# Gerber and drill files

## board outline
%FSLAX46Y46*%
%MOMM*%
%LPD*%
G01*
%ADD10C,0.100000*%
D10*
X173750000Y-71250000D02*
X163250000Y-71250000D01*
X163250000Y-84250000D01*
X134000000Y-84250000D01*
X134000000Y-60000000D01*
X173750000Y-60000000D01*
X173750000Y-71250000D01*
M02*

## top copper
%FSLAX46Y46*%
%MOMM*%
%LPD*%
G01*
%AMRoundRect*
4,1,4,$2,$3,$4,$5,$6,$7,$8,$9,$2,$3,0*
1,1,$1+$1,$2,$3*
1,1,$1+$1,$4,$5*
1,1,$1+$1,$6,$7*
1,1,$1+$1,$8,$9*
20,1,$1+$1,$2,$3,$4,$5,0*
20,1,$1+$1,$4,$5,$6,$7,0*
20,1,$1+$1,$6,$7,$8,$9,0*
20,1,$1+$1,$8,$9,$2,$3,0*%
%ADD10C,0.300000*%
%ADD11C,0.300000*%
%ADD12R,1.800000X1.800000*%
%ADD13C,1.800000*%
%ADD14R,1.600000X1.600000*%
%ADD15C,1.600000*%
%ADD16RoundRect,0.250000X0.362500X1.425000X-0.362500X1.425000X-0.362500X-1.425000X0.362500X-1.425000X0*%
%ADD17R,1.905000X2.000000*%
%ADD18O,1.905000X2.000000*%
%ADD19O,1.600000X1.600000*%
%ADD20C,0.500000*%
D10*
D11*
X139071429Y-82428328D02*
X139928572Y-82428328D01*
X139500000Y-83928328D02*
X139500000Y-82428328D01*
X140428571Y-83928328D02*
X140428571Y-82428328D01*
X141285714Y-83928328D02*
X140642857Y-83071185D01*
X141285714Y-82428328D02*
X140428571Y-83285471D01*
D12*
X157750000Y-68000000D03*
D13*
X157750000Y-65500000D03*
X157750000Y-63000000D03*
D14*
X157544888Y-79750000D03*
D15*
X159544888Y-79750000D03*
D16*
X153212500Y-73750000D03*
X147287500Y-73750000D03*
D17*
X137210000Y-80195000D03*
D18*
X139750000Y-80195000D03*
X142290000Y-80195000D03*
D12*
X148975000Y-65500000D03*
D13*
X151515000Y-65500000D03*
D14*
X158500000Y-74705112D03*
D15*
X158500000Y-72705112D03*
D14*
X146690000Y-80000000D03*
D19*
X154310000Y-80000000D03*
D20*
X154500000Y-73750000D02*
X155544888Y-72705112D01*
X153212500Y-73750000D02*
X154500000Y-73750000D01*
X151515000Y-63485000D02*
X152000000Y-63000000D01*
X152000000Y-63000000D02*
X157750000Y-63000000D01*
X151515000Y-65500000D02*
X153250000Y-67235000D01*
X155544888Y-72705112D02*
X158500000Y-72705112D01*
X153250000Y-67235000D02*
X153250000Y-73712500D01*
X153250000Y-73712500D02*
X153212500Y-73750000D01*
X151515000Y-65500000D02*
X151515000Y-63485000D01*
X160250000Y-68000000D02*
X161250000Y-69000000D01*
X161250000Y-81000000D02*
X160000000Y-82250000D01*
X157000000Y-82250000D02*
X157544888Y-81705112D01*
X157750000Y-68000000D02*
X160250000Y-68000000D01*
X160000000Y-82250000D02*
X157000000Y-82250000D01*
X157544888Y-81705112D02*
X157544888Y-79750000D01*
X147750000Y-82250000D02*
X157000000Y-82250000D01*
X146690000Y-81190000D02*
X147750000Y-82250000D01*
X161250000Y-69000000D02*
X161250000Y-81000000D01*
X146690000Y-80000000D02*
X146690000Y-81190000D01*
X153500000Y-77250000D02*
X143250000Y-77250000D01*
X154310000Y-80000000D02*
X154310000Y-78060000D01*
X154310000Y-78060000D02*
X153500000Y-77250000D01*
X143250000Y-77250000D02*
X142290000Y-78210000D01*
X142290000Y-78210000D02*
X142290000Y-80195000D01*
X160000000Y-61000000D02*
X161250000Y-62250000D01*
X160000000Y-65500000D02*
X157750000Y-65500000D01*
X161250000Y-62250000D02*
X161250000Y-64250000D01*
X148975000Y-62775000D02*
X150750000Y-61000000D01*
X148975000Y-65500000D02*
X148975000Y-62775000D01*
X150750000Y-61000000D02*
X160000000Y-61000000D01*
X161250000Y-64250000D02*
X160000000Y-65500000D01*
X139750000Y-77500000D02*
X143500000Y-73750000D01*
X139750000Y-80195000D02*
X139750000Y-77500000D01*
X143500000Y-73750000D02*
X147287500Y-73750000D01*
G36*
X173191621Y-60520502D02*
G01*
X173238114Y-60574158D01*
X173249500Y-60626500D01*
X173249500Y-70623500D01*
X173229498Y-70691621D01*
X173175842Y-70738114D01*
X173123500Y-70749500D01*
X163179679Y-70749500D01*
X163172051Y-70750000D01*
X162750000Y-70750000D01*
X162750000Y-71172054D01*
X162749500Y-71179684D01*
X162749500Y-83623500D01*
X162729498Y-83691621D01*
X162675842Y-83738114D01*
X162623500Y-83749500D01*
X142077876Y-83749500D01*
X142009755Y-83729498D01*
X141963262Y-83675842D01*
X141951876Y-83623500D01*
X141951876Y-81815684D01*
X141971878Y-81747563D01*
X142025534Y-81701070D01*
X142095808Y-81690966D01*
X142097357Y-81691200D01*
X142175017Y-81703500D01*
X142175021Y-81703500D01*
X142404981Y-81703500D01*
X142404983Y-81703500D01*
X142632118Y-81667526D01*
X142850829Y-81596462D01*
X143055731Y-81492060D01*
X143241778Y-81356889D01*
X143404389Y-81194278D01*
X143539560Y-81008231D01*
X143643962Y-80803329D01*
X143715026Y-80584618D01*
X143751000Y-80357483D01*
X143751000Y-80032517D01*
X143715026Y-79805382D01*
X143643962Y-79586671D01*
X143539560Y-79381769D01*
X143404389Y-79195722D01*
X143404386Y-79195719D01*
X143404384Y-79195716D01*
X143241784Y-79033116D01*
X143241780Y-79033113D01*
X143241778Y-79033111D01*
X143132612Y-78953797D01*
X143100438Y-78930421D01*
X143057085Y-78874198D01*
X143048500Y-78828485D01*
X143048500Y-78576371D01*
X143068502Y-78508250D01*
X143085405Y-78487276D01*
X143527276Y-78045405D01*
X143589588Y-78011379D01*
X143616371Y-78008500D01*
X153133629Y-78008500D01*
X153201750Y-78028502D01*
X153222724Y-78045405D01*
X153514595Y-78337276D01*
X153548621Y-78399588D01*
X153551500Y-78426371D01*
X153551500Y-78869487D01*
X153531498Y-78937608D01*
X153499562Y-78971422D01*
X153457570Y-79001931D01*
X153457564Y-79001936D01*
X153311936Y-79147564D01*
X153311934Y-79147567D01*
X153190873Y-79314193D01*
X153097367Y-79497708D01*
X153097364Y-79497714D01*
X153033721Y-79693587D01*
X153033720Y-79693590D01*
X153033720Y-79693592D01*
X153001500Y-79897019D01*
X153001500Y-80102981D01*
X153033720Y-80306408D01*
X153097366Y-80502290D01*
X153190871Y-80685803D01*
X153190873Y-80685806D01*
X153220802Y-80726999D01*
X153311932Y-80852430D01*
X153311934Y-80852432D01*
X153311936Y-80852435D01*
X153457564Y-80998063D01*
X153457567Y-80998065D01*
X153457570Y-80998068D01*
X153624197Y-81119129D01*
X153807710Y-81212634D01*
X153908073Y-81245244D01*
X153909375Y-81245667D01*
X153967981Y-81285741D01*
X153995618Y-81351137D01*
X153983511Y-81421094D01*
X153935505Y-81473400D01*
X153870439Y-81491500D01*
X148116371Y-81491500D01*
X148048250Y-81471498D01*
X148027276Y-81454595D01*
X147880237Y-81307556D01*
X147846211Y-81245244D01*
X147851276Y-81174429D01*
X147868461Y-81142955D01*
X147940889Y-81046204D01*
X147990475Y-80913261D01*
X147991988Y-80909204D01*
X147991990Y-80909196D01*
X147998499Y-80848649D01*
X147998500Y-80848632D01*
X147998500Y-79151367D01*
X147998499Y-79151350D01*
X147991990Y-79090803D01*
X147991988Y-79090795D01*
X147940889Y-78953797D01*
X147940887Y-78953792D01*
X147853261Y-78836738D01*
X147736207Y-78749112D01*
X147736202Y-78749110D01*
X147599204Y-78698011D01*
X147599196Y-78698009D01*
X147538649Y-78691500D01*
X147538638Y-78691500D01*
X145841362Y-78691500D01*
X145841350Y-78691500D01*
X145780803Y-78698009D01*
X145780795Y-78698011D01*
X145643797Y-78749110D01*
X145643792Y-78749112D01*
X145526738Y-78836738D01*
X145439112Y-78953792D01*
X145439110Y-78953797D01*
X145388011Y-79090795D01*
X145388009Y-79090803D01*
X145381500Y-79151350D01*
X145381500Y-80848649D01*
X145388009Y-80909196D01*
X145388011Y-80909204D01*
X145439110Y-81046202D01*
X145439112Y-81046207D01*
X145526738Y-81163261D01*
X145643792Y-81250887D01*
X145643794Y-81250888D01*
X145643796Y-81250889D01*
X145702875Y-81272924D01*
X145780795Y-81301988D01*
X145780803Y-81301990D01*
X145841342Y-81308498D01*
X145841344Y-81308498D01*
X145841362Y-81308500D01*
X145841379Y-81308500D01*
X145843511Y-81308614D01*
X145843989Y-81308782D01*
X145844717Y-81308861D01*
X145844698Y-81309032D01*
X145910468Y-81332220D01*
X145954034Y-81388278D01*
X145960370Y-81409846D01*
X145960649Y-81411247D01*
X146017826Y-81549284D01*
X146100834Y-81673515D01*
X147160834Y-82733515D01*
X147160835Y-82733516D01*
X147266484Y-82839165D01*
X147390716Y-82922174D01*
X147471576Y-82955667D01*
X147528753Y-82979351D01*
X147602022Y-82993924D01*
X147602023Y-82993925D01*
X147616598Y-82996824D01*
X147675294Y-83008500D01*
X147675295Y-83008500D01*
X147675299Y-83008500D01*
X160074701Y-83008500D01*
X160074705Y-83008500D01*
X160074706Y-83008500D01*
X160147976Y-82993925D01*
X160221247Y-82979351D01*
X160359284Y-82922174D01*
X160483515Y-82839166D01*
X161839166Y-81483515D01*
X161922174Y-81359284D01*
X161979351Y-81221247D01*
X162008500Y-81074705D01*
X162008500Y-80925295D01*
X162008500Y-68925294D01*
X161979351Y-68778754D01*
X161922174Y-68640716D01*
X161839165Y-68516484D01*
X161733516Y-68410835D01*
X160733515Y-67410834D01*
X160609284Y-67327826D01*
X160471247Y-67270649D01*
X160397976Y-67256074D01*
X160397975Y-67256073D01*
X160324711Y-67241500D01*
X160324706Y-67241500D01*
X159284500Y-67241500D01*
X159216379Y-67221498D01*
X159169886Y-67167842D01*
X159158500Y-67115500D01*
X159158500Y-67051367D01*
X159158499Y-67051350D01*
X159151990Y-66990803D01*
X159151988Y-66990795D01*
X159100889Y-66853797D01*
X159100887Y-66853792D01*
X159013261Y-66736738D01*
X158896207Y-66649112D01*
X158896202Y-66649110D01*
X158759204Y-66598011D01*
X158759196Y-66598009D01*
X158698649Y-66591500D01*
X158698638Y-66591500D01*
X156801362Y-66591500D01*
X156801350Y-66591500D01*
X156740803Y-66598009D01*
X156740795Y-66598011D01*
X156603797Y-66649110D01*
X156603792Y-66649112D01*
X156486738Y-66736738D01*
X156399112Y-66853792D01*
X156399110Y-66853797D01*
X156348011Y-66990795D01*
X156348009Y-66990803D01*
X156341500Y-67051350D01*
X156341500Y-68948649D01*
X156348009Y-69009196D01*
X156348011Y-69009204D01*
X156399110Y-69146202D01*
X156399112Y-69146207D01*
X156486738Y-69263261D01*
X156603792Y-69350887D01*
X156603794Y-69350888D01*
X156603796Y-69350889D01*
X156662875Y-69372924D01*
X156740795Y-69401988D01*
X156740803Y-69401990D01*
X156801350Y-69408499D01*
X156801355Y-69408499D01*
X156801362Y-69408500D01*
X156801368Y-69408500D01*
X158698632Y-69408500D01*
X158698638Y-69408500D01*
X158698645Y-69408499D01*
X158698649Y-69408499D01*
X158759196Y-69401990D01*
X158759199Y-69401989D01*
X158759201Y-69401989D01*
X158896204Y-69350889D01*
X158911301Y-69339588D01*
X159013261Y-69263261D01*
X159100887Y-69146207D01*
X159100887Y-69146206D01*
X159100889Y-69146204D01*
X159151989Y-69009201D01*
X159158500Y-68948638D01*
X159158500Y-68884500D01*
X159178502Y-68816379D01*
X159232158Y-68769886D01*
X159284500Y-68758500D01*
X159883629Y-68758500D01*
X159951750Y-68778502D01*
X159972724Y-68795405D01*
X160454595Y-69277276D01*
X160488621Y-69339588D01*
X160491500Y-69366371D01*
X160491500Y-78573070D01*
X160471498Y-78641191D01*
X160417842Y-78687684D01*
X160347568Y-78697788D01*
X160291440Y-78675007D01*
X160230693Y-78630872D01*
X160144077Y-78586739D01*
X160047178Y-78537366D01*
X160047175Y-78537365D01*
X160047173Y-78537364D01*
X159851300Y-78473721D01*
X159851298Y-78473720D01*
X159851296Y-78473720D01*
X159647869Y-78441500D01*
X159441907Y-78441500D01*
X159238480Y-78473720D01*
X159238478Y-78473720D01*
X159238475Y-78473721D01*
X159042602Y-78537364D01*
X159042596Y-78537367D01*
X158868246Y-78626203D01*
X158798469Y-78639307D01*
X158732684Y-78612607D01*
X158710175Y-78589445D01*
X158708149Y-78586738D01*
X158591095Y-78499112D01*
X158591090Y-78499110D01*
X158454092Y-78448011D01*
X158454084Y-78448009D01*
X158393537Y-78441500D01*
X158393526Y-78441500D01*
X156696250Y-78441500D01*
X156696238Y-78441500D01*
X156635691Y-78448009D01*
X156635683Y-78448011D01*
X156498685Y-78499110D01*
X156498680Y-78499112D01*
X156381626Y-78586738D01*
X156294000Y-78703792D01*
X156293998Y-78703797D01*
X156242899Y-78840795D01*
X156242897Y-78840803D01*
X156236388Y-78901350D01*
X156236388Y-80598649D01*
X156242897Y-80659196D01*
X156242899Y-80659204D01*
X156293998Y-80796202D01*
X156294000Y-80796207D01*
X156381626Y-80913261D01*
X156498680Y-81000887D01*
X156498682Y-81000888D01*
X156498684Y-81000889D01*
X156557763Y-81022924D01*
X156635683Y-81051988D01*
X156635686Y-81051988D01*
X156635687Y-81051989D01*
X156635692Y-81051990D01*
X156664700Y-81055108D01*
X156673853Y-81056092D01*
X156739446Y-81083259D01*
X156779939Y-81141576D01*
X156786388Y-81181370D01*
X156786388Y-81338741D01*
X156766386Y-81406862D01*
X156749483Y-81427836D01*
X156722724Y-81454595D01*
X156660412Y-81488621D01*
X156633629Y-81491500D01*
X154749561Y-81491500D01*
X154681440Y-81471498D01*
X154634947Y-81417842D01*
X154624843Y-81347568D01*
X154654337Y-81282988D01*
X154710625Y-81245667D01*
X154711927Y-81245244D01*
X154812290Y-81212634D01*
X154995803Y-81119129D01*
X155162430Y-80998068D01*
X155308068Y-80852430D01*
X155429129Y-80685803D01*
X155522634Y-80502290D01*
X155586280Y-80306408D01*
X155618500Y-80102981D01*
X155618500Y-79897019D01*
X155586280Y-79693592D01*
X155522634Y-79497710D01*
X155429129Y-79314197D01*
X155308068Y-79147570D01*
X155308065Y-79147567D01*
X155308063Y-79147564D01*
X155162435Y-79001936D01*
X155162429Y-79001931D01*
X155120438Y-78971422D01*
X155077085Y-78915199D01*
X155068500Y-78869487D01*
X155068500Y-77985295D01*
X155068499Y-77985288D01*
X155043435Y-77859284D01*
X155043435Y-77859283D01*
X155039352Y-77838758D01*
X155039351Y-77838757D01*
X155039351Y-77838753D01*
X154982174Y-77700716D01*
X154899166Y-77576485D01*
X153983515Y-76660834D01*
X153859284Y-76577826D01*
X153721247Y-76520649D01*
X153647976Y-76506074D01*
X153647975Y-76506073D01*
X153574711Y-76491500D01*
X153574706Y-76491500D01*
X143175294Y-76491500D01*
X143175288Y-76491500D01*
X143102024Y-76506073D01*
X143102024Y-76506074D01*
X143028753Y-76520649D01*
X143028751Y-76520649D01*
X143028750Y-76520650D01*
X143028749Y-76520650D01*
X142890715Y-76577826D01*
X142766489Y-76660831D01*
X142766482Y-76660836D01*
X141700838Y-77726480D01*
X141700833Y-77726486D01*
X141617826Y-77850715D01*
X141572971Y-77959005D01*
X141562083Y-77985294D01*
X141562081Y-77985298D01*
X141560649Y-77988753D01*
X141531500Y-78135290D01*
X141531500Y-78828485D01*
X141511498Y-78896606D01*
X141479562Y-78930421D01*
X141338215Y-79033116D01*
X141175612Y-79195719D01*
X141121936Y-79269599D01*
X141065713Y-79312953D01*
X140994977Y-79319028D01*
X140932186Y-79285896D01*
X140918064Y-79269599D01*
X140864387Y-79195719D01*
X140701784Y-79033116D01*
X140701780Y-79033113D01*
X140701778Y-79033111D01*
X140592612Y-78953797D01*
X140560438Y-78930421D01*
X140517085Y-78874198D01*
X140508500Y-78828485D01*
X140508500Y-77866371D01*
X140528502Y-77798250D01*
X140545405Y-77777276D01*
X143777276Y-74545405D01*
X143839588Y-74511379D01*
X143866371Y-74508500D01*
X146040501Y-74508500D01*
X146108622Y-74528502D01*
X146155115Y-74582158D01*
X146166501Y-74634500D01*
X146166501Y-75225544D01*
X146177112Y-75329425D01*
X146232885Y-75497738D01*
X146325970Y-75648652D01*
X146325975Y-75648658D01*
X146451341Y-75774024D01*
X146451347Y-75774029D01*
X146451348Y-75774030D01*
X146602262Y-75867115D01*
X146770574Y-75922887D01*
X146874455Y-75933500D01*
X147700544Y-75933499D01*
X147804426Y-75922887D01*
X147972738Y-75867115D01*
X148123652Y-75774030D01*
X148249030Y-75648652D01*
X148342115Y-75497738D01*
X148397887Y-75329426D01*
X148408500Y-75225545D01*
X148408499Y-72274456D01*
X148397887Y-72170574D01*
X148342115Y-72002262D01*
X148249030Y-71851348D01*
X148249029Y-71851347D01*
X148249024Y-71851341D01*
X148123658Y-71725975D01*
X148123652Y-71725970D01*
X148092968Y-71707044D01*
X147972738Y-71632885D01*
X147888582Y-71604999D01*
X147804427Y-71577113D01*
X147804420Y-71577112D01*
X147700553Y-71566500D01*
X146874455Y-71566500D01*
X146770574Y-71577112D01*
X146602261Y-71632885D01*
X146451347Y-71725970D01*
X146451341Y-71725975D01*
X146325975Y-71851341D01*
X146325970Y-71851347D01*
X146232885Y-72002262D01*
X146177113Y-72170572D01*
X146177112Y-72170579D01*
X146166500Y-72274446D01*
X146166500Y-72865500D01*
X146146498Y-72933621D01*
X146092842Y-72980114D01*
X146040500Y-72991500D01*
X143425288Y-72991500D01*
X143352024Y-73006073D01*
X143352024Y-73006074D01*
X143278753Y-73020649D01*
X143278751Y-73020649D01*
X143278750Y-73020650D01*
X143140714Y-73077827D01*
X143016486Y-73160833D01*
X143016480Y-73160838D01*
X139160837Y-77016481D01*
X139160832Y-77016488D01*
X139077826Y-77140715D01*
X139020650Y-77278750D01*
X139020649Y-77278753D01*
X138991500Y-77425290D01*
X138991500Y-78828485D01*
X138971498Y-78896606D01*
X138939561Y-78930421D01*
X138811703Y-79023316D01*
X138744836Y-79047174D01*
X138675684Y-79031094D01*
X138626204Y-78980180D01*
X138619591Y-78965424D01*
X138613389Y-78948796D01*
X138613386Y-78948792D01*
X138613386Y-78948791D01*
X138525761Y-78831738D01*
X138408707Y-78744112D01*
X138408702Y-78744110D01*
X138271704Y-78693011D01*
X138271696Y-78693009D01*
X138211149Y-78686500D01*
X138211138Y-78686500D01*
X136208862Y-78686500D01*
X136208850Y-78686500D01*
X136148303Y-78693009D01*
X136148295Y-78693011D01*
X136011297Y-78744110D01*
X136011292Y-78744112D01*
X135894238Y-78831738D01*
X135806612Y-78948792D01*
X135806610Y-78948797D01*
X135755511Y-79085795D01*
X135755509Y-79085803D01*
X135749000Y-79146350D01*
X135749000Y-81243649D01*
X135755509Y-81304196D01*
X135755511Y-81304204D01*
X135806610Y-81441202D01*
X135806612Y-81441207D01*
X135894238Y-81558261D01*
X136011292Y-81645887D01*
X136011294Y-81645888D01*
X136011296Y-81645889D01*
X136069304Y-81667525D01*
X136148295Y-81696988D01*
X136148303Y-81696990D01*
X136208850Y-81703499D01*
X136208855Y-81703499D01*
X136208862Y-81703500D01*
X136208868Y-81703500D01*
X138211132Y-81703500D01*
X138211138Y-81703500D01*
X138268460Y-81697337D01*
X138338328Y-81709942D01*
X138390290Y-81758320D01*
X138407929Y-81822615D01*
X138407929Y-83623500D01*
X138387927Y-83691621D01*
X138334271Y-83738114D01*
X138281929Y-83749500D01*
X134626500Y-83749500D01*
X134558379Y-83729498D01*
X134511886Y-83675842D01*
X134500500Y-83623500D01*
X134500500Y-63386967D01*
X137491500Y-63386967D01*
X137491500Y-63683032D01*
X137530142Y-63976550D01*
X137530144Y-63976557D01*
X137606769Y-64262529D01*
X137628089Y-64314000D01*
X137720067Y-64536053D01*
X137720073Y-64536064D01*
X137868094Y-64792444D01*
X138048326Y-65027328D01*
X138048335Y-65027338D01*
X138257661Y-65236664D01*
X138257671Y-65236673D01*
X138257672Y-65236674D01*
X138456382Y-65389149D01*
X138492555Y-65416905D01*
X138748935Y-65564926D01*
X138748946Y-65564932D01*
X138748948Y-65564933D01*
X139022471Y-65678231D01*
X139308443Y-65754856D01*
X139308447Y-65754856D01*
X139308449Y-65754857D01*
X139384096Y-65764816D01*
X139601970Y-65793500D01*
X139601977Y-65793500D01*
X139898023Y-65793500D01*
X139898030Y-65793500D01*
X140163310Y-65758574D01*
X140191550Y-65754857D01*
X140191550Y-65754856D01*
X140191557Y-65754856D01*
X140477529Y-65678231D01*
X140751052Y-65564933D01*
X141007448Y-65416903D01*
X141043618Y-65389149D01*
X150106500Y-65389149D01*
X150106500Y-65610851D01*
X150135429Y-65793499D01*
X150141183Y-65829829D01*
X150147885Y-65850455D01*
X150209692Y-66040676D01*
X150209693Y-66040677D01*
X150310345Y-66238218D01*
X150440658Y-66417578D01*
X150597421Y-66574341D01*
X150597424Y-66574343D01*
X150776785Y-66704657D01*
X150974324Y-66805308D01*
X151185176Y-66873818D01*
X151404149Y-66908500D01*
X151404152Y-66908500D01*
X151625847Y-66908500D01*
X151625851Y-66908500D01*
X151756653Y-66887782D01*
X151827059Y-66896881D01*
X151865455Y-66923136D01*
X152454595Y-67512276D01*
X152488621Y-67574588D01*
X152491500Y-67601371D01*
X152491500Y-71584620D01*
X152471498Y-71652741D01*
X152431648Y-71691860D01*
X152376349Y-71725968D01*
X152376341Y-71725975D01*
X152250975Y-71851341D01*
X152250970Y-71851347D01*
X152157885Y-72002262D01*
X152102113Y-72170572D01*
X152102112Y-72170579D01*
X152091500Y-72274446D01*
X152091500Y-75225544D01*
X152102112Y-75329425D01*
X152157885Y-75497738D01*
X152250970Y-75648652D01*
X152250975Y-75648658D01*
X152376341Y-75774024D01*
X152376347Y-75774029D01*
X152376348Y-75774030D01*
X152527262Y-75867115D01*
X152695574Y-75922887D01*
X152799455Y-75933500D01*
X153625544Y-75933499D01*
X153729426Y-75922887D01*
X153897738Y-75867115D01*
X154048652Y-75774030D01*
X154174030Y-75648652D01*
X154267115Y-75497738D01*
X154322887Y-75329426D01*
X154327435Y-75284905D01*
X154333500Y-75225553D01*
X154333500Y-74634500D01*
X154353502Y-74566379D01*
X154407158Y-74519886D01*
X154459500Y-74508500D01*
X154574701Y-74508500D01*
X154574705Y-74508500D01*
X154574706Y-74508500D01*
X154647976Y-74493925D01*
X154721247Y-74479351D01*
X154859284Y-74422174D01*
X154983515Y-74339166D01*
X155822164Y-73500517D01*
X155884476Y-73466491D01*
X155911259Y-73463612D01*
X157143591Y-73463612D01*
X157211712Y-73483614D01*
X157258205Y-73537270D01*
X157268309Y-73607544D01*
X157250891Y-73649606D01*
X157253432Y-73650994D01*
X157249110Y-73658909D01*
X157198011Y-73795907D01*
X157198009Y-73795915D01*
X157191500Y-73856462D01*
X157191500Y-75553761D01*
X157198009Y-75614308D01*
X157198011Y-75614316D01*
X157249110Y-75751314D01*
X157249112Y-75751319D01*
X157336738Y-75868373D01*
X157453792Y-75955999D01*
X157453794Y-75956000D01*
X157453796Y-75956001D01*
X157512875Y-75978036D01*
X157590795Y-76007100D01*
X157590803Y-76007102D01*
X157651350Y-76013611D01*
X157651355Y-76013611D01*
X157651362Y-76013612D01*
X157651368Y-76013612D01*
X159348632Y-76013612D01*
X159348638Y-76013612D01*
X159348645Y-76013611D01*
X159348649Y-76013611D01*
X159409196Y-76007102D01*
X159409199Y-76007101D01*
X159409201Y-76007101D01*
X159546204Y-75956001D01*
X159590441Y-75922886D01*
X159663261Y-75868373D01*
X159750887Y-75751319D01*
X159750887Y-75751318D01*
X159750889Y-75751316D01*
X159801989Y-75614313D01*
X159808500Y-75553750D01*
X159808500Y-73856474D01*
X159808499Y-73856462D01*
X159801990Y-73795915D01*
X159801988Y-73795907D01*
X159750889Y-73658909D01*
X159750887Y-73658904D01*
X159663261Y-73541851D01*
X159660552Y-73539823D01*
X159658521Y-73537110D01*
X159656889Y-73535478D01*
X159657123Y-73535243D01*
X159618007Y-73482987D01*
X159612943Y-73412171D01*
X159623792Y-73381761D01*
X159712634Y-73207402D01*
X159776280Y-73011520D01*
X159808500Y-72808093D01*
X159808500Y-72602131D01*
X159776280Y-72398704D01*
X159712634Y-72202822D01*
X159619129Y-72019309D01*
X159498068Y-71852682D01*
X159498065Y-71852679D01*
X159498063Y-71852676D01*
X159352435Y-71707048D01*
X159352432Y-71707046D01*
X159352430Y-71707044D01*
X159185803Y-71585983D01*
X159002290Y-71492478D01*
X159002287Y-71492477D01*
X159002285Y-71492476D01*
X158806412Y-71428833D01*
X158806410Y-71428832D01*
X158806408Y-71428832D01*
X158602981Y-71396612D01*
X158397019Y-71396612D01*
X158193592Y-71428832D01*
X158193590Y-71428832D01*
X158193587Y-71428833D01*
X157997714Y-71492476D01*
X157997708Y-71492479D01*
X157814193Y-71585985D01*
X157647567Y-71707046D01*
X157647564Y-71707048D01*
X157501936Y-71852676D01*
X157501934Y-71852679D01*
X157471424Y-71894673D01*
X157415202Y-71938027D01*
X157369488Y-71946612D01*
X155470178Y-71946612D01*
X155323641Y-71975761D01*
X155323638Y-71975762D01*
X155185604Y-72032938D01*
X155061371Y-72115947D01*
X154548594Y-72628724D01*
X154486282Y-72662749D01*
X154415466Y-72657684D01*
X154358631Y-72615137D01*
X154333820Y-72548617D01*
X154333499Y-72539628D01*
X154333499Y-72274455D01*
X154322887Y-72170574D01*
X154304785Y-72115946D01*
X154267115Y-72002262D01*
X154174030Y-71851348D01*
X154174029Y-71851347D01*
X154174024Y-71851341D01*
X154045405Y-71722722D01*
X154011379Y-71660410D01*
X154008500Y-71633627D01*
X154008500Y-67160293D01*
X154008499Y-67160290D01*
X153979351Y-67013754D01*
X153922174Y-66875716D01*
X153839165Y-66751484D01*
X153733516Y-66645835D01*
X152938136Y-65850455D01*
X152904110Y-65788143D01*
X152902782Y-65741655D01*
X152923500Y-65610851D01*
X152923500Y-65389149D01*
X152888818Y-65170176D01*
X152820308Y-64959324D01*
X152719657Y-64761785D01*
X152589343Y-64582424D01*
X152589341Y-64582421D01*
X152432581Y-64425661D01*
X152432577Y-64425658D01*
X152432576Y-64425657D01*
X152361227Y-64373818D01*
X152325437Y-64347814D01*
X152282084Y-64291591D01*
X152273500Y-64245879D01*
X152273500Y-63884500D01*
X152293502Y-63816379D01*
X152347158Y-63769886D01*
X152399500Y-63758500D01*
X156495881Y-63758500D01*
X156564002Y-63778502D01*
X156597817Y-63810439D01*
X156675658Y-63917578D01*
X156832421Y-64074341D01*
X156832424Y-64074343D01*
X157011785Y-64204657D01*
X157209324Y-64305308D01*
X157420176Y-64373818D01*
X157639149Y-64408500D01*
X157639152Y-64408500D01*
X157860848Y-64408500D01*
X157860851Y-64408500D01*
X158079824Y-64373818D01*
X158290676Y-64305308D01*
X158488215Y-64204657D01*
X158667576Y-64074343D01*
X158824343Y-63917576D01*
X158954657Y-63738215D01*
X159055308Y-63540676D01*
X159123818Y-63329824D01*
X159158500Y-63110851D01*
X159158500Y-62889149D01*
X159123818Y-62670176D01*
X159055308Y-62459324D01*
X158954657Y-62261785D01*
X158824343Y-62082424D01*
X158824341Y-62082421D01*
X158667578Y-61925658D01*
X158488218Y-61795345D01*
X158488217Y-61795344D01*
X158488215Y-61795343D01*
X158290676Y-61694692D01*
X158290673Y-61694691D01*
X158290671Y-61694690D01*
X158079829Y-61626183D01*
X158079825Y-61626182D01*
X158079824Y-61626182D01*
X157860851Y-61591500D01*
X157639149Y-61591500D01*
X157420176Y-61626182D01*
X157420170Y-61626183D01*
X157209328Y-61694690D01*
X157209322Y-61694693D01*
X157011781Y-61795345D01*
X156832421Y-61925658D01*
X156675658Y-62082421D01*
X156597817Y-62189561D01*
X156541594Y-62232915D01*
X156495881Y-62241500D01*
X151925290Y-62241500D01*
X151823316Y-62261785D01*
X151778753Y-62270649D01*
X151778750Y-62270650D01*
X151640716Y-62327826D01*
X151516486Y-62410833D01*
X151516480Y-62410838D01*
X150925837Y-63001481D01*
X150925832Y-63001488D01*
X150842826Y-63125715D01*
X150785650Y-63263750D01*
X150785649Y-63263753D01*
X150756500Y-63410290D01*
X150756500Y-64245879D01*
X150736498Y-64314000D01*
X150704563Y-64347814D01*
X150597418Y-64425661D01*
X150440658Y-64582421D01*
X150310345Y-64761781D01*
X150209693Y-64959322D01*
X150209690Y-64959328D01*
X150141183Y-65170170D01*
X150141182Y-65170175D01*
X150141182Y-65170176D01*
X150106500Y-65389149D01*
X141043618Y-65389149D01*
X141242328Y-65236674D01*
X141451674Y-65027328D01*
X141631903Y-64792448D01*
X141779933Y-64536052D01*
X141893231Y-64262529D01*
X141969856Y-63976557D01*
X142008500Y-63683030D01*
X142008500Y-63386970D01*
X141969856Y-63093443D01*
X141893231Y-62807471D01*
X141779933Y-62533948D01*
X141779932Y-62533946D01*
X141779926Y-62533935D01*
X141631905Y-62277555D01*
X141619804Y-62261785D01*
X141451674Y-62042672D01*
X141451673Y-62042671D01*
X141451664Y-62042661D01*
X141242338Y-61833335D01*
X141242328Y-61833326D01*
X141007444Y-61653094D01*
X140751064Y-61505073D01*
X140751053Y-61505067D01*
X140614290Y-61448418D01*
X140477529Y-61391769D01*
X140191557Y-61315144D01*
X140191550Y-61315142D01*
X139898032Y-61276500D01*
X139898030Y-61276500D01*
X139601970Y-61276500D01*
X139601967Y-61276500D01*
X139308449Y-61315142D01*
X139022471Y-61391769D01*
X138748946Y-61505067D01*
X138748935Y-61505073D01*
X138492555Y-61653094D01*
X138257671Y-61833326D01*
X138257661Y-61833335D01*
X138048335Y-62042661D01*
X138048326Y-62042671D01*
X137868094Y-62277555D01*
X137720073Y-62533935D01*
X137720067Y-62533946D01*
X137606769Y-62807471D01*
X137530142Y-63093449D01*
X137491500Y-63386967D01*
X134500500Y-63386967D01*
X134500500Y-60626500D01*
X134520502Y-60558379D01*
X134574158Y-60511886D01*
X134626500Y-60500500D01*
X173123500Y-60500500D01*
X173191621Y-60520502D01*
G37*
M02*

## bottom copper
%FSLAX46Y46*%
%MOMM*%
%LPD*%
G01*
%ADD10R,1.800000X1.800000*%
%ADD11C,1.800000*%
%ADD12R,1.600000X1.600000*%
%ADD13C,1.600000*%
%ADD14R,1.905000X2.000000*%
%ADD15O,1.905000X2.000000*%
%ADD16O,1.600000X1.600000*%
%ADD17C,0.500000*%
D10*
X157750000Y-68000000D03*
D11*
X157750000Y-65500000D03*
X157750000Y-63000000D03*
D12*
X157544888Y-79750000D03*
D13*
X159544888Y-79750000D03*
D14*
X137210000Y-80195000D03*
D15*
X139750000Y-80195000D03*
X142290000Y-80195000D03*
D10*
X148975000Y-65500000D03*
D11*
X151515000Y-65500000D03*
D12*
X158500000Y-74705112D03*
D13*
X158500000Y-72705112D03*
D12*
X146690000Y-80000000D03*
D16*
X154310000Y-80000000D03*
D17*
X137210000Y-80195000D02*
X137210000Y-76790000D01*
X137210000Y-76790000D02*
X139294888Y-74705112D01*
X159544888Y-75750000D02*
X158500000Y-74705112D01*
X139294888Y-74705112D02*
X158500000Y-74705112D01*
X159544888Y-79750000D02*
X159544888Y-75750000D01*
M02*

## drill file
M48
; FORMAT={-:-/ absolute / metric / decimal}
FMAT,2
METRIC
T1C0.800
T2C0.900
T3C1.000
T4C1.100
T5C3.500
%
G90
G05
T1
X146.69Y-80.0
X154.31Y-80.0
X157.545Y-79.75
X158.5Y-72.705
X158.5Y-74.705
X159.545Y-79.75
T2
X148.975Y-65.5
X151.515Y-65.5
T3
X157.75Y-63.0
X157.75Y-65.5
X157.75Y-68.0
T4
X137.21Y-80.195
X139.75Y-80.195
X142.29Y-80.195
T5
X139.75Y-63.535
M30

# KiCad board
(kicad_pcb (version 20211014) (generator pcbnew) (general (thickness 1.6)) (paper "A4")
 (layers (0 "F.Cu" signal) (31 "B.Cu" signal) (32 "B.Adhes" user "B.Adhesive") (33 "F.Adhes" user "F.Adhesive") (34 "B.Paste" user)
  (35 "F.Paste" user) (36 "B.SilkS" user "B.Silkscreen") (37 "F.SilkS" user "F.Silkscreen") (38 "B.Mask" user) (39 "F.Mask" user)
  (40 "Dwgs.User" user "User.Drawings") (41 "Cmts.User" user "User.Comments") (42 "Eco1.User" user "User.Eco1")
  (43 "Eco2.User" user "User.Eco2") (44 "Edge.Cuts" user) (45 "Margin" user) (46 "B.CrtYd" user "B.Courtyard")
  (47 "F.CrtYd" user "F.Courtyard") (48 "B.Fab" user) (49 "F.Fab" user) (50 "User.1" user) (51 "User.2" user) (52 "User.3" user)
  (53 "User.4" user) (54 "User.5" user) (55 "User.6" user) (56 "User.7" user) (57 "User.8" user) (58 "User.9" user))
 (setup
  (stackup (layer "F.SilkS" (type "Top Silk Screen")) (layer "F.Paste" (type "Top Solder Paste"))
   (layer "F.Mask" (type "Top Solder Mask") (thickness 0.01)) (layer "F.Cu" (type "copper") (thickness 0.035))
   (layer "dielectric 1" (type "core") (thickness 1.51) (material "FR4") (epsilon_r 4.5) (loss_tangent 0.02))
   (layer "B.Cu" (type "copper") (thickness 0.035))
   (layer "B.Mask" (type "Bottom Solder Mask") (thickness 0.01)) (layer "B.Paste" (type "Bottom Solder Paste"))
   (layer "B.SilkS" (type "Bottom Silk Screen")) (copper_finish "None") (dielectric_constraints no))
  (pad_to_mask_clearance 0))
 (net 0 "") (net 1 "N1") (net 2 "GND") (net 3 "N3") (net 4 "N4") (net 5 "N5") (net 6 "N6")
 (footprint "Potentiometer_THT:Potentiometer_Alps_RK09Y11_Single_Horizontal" (layer "F.Cu") (at 157.75 68 180)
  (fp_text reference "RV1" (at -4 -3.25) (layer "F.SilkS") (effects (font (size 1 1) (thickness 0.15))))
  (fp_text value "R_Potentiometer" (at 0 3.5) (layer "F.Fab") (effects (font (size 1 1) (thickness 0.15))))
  (pad "1" thru_hole rect (at 0 0) (size 1.8 1.8) (drill 1) (layers *.Cu *.Mask) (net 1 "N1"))
  (pad "2" thru_hole circle (at 0 2.5) (size 1.8 1.8) (drill 1) (layers *.Cu *.Mask) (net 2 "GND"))
  (pad "3" thru_hole circle (at 0 5) (size 1.8 1.8) (drill 1) (layers *.Cu *.Mask) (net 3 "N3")))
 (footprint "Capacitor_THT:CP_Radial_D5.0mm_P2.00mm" (layer "F.Cu") (at 157.544888 79.75)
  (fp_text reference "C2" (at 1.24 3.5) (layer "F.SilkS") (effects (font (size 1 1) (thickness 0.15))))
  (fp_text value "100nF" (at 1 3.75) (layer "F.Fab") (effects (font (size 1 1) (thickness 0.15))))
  (pad "1" thru_hole rect (at 0 0) (size 1.6 1.6) (drill 0.8) (layers *.Cu *.Mask) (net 1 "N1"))
  (pad "2" thru_hole circle (at 2 0) (size 1.6 1.6) (drill 0.8) (layers *.Cu *.Mask) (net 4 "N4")))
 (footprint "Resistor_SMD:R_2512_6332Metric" (layer "F.Cu") (at 150.25 73.75 180)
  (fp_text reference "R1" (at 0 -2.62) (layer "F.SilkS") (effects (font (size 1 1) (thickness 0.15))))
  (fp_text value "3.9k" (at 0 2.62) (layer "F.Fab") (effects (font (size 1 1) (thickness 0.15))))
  (pad "1" smd roundrect (at -2.9625 0 180) (size 1.225 3.35) (layers "F.Cu" "F.Paste" "F.Mask") (roundrect_rratio 0.2040816327)
   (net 3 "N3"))
  (pad "2" smd roundrect (at 2.9625 0 180) (size 1.225 3.35) (layers "F.Cu" "F.Paste" "F.Mask") (roundrect_rratio 0.2040816327) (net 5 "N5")))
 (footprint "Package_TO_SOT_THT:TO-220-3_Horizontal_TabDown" (layer "F.Cu") (at 137.21 80.195)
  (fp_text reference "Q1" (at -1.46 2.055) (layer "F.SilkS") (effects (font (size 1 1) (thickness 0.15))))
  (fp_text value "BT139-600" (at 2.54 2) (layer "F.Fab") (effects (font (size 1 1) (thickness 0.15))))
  (pad "" np_thru_hole oval (at 2.54 -16.66) (size 3.5 3.5) (drill 3.5) (layers *.Cu *.Mask))
  (pad "1" thru_hole rect (at 0 0) (size 1.905 2) (drill 1.1) (layers *.Cu *.Mask) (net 4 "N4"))
  (pad "2" thru_hole oval (at 2.54 0) (size 1.905 2) (drill 1.1) (layers *.Cu *.Mask) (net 5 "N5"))
  (pad "3" thru_hole oval (at 5.08 0) (size 1.905 2) (drill 1.1) (layers *.Cu *.Mask) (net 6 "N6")))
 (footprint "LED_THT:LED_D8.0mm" (layer "F.Cu") (at 148.975 65.5)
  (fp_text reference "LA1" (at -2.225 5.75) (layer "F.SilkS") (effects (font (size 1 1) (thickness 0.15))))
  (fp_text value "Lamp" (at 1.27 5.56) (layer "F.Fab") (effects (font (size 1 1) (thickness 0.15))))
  (pad "1" thru_hole rect (at 0 0) (size 1.8 1.8) (drill 0.9) (layers *.Cu *.Mask) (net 2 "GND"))
  (pad "2" thru_hole circle (at 2.54 0) (size 1.8 1.8) (drill 0.9) (layers *.Cu *.Mask) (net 3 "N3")))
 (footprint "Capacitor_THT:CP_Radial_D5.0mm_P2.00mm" (layer "F.Cu") (at 158.5 74.705112 90)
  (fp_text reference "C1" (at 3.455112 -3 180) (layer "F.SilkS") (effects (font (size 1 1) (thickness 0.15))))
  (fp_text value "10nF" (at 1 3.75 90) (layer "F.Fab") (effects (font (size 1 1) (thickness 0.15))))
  (pad "1" thru_hole rect (at 0 0 90) (size 1.6 1.6) (drill 0.8) (layers *.Cu *.Mask) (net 4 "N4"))
  (pad "2" thru_hole circle (at 2 0 90) (size 1.6 1.6) (drill 0.8) (layers *.Cu *.Mask) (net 3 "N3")))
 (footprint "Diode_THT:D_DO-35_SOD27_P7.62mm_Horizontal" (layer "F.Cu") (at 146.69 80)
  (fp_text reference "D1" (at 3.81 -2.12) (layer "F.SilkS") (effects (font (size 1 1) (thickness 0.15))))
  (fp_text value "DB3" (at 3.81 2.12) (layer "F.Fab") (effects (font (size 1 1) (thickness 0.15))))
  (pad "1" thru_hole rect (at 0 0) (size 1.6 1.6) (drill 0.8) (layers *.Cu *.Mask) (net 1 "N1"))
  (pad "2" thru_hole oval (at 7.62 0) (size 1.6 1.6) (drill 0.8) (layers *.Cu *.Mask) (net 6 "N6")))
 (gr_poly
  (pts (xy 173.75 71.25) (xy 163.25 71.25) (xy 163.25 84.25) (xy 134 84.25) (xy 134 60) (xy 173.75 60)) (layer "Edge.Cuts") (width 0.1)
  (fill none))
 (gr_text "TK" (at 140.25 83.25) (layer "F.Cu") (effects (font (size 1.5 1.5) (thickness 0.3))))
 (segment (start 137.21 80.195) (end 137.21 76.79) (width 0.5) (layer "B.Cu") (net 4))
 (segment (start 137.21 76.79) (end 139.294888 74.705112) (width 0.5) (layer "B.Cu") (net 4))
 (segment (start 159.544888 75.75) (end 158.5 74.705112) (width 0.5) (layer "B.Cu") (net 4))
 (segment (start 139.294888 74.705112) (end 158.5 74.705112) (width 0.5) (layer "B.Cu") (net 4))
 (segment (start 159.544888 79.75) (end 159.544888 75.75) (width 0.5) (layer "B.Cu") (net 4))
 (segment (start 154.5 73.75) (end 155.544888 72.705112) (width 0.5) (layer "F.Cu") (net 3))
 (segment (start 153.2125 73.75) (end 154.5 73.75) (width 0.5) (layer "F.Cu") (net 3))
 (segment (start 151.515 63.485) (end 152 63) (width 0.5) (layer "F.Cu") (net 3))
 (segment (start 152 63) (end 157.75 63) (width 0.5) (layer "F.Cu") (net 3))
 (segment (start 151.515 65.5) (end 153.25 67.235) (width 0.5) (layer "F.Cu") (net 3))
 (segment (start 155.544888 72.705112) (end 158.5 72.705112) (width 0.5) (layer "F.Cu") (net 3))
 (segment (start 153.25 67.235) (end 153.25 73.7125) (width 0.5) (layer "F.Cu") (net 3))
 (segment (start 153.25 73.7125) (end 153.2125 73.75) (width 0.5) (layer "F.Cu") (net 3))
 (segment (start 151.515 65.5) (end 151.515 63.485) (width 0.5) (layer "F.Cu") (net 3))
 (segment (start 160.25 68) (end 161.25 69) (width 0.5) (layer "F.Cu") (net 1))
 (segment (start 161.25 81) (end 160 82.25) (width 0.5) (layer "F.Cu") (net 1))
 (segment (start 157 82.25) (end 157.544888 81.705112) (width 0.5) (layer "F.Cu") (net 1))
 (segment (start 157.75 68) (end 160.25 68) (width 0.5) (layer "F.Cu") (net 1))
 (segment (start 160 82.25) (end 157 82.25) (width 0.5) (layer "F.Cu") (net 1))
 (segment (start 157.544888 81.705112) (end 157.544888 79.75) (width 0.5) (layer "F.Cu") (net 1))
 (segment (start 147.75 82.25) (end 157 82.25) (width 0.5) (layer "F.Cu") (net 1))
 (segment (start 146.69 81.19) (end 147.75 82.25) (width 0.5) (layer "F.Cu") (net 1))
 (segment (start 161.25 69) (end 161.25 81) (width 0.5) (layer "F.Cu") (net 1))
 (segment (start 146.69 80) (end 146.69 81.19) (width 0.5) (layer "F.Cu") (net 1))
 (segment (start 153.5 77.25) (end 143.25 77.25) (width 0.5) (layer "F.Cu") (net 6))
 (segment (start 154.31 80) (end 154.31 78.06) (width 0.5) (layer "F.Cu") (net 6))
 (segment (start 154.31 78.06) (end 153.5 77.25) (width 0.5) (layer "F.Cu") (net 6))
 (segment (start 143.25 77.25) (end 142.29 78.21) (width 0.5) (layer "F.Cu") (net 6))
 (segment (start 142.29 78.21) (end 142.29 80.195) (width 0.5) (layer "F.Cu") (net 6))
 (segment (start 160 61) (end 161.25 62.25) (width 0.5) (layer "F.Cu") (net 2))
 (segment (start 160 65.5) (end 157.75 65.5) (width 0.5) (layer "F.Cu") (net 2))
 (segment (start 161.25 62.25) (end 161.25 64.25) (width 0.5) (layer "F.Cu") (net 2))
 (segment (start 148.975 62.775) (end 150.75 61) (width 0.5) (layer "F.Cu") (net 2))
 (segment (start 148.975 65.5) (end 148.975 62.775) (width 0.5) (layer "F.Cu") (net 2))
 (segment (start 150.75 61) (end 160 61) (width 0.5) (layer "F.Cu") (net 2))
 (segment (start 161.25 64.25) (end 160 65.5) (width 0.5) (layer "F.Cu") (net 2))
 (segment (start 139.75 77.5) (end 143.5 73.75) (width 0.5) (layer "F.Cu") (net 5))
 (segment (start 139.75 80.195) (end 139.75 77.5) (width 0.5) (layer "F.Cu") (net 5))
 (segment (start 143.5 73.75) (end 147.2875 73.75) (width 0.5) (layer "F.Cu") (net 5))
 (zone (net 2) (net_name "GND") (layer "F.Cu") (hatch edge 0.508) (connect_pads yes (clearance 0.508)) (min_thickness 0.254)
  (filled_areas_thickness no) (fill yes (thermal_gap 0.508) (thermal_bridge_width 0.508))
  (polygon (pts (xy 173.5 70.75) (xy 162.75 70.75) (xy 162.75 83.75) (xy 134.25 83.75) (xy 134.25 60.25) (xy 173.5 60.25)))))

